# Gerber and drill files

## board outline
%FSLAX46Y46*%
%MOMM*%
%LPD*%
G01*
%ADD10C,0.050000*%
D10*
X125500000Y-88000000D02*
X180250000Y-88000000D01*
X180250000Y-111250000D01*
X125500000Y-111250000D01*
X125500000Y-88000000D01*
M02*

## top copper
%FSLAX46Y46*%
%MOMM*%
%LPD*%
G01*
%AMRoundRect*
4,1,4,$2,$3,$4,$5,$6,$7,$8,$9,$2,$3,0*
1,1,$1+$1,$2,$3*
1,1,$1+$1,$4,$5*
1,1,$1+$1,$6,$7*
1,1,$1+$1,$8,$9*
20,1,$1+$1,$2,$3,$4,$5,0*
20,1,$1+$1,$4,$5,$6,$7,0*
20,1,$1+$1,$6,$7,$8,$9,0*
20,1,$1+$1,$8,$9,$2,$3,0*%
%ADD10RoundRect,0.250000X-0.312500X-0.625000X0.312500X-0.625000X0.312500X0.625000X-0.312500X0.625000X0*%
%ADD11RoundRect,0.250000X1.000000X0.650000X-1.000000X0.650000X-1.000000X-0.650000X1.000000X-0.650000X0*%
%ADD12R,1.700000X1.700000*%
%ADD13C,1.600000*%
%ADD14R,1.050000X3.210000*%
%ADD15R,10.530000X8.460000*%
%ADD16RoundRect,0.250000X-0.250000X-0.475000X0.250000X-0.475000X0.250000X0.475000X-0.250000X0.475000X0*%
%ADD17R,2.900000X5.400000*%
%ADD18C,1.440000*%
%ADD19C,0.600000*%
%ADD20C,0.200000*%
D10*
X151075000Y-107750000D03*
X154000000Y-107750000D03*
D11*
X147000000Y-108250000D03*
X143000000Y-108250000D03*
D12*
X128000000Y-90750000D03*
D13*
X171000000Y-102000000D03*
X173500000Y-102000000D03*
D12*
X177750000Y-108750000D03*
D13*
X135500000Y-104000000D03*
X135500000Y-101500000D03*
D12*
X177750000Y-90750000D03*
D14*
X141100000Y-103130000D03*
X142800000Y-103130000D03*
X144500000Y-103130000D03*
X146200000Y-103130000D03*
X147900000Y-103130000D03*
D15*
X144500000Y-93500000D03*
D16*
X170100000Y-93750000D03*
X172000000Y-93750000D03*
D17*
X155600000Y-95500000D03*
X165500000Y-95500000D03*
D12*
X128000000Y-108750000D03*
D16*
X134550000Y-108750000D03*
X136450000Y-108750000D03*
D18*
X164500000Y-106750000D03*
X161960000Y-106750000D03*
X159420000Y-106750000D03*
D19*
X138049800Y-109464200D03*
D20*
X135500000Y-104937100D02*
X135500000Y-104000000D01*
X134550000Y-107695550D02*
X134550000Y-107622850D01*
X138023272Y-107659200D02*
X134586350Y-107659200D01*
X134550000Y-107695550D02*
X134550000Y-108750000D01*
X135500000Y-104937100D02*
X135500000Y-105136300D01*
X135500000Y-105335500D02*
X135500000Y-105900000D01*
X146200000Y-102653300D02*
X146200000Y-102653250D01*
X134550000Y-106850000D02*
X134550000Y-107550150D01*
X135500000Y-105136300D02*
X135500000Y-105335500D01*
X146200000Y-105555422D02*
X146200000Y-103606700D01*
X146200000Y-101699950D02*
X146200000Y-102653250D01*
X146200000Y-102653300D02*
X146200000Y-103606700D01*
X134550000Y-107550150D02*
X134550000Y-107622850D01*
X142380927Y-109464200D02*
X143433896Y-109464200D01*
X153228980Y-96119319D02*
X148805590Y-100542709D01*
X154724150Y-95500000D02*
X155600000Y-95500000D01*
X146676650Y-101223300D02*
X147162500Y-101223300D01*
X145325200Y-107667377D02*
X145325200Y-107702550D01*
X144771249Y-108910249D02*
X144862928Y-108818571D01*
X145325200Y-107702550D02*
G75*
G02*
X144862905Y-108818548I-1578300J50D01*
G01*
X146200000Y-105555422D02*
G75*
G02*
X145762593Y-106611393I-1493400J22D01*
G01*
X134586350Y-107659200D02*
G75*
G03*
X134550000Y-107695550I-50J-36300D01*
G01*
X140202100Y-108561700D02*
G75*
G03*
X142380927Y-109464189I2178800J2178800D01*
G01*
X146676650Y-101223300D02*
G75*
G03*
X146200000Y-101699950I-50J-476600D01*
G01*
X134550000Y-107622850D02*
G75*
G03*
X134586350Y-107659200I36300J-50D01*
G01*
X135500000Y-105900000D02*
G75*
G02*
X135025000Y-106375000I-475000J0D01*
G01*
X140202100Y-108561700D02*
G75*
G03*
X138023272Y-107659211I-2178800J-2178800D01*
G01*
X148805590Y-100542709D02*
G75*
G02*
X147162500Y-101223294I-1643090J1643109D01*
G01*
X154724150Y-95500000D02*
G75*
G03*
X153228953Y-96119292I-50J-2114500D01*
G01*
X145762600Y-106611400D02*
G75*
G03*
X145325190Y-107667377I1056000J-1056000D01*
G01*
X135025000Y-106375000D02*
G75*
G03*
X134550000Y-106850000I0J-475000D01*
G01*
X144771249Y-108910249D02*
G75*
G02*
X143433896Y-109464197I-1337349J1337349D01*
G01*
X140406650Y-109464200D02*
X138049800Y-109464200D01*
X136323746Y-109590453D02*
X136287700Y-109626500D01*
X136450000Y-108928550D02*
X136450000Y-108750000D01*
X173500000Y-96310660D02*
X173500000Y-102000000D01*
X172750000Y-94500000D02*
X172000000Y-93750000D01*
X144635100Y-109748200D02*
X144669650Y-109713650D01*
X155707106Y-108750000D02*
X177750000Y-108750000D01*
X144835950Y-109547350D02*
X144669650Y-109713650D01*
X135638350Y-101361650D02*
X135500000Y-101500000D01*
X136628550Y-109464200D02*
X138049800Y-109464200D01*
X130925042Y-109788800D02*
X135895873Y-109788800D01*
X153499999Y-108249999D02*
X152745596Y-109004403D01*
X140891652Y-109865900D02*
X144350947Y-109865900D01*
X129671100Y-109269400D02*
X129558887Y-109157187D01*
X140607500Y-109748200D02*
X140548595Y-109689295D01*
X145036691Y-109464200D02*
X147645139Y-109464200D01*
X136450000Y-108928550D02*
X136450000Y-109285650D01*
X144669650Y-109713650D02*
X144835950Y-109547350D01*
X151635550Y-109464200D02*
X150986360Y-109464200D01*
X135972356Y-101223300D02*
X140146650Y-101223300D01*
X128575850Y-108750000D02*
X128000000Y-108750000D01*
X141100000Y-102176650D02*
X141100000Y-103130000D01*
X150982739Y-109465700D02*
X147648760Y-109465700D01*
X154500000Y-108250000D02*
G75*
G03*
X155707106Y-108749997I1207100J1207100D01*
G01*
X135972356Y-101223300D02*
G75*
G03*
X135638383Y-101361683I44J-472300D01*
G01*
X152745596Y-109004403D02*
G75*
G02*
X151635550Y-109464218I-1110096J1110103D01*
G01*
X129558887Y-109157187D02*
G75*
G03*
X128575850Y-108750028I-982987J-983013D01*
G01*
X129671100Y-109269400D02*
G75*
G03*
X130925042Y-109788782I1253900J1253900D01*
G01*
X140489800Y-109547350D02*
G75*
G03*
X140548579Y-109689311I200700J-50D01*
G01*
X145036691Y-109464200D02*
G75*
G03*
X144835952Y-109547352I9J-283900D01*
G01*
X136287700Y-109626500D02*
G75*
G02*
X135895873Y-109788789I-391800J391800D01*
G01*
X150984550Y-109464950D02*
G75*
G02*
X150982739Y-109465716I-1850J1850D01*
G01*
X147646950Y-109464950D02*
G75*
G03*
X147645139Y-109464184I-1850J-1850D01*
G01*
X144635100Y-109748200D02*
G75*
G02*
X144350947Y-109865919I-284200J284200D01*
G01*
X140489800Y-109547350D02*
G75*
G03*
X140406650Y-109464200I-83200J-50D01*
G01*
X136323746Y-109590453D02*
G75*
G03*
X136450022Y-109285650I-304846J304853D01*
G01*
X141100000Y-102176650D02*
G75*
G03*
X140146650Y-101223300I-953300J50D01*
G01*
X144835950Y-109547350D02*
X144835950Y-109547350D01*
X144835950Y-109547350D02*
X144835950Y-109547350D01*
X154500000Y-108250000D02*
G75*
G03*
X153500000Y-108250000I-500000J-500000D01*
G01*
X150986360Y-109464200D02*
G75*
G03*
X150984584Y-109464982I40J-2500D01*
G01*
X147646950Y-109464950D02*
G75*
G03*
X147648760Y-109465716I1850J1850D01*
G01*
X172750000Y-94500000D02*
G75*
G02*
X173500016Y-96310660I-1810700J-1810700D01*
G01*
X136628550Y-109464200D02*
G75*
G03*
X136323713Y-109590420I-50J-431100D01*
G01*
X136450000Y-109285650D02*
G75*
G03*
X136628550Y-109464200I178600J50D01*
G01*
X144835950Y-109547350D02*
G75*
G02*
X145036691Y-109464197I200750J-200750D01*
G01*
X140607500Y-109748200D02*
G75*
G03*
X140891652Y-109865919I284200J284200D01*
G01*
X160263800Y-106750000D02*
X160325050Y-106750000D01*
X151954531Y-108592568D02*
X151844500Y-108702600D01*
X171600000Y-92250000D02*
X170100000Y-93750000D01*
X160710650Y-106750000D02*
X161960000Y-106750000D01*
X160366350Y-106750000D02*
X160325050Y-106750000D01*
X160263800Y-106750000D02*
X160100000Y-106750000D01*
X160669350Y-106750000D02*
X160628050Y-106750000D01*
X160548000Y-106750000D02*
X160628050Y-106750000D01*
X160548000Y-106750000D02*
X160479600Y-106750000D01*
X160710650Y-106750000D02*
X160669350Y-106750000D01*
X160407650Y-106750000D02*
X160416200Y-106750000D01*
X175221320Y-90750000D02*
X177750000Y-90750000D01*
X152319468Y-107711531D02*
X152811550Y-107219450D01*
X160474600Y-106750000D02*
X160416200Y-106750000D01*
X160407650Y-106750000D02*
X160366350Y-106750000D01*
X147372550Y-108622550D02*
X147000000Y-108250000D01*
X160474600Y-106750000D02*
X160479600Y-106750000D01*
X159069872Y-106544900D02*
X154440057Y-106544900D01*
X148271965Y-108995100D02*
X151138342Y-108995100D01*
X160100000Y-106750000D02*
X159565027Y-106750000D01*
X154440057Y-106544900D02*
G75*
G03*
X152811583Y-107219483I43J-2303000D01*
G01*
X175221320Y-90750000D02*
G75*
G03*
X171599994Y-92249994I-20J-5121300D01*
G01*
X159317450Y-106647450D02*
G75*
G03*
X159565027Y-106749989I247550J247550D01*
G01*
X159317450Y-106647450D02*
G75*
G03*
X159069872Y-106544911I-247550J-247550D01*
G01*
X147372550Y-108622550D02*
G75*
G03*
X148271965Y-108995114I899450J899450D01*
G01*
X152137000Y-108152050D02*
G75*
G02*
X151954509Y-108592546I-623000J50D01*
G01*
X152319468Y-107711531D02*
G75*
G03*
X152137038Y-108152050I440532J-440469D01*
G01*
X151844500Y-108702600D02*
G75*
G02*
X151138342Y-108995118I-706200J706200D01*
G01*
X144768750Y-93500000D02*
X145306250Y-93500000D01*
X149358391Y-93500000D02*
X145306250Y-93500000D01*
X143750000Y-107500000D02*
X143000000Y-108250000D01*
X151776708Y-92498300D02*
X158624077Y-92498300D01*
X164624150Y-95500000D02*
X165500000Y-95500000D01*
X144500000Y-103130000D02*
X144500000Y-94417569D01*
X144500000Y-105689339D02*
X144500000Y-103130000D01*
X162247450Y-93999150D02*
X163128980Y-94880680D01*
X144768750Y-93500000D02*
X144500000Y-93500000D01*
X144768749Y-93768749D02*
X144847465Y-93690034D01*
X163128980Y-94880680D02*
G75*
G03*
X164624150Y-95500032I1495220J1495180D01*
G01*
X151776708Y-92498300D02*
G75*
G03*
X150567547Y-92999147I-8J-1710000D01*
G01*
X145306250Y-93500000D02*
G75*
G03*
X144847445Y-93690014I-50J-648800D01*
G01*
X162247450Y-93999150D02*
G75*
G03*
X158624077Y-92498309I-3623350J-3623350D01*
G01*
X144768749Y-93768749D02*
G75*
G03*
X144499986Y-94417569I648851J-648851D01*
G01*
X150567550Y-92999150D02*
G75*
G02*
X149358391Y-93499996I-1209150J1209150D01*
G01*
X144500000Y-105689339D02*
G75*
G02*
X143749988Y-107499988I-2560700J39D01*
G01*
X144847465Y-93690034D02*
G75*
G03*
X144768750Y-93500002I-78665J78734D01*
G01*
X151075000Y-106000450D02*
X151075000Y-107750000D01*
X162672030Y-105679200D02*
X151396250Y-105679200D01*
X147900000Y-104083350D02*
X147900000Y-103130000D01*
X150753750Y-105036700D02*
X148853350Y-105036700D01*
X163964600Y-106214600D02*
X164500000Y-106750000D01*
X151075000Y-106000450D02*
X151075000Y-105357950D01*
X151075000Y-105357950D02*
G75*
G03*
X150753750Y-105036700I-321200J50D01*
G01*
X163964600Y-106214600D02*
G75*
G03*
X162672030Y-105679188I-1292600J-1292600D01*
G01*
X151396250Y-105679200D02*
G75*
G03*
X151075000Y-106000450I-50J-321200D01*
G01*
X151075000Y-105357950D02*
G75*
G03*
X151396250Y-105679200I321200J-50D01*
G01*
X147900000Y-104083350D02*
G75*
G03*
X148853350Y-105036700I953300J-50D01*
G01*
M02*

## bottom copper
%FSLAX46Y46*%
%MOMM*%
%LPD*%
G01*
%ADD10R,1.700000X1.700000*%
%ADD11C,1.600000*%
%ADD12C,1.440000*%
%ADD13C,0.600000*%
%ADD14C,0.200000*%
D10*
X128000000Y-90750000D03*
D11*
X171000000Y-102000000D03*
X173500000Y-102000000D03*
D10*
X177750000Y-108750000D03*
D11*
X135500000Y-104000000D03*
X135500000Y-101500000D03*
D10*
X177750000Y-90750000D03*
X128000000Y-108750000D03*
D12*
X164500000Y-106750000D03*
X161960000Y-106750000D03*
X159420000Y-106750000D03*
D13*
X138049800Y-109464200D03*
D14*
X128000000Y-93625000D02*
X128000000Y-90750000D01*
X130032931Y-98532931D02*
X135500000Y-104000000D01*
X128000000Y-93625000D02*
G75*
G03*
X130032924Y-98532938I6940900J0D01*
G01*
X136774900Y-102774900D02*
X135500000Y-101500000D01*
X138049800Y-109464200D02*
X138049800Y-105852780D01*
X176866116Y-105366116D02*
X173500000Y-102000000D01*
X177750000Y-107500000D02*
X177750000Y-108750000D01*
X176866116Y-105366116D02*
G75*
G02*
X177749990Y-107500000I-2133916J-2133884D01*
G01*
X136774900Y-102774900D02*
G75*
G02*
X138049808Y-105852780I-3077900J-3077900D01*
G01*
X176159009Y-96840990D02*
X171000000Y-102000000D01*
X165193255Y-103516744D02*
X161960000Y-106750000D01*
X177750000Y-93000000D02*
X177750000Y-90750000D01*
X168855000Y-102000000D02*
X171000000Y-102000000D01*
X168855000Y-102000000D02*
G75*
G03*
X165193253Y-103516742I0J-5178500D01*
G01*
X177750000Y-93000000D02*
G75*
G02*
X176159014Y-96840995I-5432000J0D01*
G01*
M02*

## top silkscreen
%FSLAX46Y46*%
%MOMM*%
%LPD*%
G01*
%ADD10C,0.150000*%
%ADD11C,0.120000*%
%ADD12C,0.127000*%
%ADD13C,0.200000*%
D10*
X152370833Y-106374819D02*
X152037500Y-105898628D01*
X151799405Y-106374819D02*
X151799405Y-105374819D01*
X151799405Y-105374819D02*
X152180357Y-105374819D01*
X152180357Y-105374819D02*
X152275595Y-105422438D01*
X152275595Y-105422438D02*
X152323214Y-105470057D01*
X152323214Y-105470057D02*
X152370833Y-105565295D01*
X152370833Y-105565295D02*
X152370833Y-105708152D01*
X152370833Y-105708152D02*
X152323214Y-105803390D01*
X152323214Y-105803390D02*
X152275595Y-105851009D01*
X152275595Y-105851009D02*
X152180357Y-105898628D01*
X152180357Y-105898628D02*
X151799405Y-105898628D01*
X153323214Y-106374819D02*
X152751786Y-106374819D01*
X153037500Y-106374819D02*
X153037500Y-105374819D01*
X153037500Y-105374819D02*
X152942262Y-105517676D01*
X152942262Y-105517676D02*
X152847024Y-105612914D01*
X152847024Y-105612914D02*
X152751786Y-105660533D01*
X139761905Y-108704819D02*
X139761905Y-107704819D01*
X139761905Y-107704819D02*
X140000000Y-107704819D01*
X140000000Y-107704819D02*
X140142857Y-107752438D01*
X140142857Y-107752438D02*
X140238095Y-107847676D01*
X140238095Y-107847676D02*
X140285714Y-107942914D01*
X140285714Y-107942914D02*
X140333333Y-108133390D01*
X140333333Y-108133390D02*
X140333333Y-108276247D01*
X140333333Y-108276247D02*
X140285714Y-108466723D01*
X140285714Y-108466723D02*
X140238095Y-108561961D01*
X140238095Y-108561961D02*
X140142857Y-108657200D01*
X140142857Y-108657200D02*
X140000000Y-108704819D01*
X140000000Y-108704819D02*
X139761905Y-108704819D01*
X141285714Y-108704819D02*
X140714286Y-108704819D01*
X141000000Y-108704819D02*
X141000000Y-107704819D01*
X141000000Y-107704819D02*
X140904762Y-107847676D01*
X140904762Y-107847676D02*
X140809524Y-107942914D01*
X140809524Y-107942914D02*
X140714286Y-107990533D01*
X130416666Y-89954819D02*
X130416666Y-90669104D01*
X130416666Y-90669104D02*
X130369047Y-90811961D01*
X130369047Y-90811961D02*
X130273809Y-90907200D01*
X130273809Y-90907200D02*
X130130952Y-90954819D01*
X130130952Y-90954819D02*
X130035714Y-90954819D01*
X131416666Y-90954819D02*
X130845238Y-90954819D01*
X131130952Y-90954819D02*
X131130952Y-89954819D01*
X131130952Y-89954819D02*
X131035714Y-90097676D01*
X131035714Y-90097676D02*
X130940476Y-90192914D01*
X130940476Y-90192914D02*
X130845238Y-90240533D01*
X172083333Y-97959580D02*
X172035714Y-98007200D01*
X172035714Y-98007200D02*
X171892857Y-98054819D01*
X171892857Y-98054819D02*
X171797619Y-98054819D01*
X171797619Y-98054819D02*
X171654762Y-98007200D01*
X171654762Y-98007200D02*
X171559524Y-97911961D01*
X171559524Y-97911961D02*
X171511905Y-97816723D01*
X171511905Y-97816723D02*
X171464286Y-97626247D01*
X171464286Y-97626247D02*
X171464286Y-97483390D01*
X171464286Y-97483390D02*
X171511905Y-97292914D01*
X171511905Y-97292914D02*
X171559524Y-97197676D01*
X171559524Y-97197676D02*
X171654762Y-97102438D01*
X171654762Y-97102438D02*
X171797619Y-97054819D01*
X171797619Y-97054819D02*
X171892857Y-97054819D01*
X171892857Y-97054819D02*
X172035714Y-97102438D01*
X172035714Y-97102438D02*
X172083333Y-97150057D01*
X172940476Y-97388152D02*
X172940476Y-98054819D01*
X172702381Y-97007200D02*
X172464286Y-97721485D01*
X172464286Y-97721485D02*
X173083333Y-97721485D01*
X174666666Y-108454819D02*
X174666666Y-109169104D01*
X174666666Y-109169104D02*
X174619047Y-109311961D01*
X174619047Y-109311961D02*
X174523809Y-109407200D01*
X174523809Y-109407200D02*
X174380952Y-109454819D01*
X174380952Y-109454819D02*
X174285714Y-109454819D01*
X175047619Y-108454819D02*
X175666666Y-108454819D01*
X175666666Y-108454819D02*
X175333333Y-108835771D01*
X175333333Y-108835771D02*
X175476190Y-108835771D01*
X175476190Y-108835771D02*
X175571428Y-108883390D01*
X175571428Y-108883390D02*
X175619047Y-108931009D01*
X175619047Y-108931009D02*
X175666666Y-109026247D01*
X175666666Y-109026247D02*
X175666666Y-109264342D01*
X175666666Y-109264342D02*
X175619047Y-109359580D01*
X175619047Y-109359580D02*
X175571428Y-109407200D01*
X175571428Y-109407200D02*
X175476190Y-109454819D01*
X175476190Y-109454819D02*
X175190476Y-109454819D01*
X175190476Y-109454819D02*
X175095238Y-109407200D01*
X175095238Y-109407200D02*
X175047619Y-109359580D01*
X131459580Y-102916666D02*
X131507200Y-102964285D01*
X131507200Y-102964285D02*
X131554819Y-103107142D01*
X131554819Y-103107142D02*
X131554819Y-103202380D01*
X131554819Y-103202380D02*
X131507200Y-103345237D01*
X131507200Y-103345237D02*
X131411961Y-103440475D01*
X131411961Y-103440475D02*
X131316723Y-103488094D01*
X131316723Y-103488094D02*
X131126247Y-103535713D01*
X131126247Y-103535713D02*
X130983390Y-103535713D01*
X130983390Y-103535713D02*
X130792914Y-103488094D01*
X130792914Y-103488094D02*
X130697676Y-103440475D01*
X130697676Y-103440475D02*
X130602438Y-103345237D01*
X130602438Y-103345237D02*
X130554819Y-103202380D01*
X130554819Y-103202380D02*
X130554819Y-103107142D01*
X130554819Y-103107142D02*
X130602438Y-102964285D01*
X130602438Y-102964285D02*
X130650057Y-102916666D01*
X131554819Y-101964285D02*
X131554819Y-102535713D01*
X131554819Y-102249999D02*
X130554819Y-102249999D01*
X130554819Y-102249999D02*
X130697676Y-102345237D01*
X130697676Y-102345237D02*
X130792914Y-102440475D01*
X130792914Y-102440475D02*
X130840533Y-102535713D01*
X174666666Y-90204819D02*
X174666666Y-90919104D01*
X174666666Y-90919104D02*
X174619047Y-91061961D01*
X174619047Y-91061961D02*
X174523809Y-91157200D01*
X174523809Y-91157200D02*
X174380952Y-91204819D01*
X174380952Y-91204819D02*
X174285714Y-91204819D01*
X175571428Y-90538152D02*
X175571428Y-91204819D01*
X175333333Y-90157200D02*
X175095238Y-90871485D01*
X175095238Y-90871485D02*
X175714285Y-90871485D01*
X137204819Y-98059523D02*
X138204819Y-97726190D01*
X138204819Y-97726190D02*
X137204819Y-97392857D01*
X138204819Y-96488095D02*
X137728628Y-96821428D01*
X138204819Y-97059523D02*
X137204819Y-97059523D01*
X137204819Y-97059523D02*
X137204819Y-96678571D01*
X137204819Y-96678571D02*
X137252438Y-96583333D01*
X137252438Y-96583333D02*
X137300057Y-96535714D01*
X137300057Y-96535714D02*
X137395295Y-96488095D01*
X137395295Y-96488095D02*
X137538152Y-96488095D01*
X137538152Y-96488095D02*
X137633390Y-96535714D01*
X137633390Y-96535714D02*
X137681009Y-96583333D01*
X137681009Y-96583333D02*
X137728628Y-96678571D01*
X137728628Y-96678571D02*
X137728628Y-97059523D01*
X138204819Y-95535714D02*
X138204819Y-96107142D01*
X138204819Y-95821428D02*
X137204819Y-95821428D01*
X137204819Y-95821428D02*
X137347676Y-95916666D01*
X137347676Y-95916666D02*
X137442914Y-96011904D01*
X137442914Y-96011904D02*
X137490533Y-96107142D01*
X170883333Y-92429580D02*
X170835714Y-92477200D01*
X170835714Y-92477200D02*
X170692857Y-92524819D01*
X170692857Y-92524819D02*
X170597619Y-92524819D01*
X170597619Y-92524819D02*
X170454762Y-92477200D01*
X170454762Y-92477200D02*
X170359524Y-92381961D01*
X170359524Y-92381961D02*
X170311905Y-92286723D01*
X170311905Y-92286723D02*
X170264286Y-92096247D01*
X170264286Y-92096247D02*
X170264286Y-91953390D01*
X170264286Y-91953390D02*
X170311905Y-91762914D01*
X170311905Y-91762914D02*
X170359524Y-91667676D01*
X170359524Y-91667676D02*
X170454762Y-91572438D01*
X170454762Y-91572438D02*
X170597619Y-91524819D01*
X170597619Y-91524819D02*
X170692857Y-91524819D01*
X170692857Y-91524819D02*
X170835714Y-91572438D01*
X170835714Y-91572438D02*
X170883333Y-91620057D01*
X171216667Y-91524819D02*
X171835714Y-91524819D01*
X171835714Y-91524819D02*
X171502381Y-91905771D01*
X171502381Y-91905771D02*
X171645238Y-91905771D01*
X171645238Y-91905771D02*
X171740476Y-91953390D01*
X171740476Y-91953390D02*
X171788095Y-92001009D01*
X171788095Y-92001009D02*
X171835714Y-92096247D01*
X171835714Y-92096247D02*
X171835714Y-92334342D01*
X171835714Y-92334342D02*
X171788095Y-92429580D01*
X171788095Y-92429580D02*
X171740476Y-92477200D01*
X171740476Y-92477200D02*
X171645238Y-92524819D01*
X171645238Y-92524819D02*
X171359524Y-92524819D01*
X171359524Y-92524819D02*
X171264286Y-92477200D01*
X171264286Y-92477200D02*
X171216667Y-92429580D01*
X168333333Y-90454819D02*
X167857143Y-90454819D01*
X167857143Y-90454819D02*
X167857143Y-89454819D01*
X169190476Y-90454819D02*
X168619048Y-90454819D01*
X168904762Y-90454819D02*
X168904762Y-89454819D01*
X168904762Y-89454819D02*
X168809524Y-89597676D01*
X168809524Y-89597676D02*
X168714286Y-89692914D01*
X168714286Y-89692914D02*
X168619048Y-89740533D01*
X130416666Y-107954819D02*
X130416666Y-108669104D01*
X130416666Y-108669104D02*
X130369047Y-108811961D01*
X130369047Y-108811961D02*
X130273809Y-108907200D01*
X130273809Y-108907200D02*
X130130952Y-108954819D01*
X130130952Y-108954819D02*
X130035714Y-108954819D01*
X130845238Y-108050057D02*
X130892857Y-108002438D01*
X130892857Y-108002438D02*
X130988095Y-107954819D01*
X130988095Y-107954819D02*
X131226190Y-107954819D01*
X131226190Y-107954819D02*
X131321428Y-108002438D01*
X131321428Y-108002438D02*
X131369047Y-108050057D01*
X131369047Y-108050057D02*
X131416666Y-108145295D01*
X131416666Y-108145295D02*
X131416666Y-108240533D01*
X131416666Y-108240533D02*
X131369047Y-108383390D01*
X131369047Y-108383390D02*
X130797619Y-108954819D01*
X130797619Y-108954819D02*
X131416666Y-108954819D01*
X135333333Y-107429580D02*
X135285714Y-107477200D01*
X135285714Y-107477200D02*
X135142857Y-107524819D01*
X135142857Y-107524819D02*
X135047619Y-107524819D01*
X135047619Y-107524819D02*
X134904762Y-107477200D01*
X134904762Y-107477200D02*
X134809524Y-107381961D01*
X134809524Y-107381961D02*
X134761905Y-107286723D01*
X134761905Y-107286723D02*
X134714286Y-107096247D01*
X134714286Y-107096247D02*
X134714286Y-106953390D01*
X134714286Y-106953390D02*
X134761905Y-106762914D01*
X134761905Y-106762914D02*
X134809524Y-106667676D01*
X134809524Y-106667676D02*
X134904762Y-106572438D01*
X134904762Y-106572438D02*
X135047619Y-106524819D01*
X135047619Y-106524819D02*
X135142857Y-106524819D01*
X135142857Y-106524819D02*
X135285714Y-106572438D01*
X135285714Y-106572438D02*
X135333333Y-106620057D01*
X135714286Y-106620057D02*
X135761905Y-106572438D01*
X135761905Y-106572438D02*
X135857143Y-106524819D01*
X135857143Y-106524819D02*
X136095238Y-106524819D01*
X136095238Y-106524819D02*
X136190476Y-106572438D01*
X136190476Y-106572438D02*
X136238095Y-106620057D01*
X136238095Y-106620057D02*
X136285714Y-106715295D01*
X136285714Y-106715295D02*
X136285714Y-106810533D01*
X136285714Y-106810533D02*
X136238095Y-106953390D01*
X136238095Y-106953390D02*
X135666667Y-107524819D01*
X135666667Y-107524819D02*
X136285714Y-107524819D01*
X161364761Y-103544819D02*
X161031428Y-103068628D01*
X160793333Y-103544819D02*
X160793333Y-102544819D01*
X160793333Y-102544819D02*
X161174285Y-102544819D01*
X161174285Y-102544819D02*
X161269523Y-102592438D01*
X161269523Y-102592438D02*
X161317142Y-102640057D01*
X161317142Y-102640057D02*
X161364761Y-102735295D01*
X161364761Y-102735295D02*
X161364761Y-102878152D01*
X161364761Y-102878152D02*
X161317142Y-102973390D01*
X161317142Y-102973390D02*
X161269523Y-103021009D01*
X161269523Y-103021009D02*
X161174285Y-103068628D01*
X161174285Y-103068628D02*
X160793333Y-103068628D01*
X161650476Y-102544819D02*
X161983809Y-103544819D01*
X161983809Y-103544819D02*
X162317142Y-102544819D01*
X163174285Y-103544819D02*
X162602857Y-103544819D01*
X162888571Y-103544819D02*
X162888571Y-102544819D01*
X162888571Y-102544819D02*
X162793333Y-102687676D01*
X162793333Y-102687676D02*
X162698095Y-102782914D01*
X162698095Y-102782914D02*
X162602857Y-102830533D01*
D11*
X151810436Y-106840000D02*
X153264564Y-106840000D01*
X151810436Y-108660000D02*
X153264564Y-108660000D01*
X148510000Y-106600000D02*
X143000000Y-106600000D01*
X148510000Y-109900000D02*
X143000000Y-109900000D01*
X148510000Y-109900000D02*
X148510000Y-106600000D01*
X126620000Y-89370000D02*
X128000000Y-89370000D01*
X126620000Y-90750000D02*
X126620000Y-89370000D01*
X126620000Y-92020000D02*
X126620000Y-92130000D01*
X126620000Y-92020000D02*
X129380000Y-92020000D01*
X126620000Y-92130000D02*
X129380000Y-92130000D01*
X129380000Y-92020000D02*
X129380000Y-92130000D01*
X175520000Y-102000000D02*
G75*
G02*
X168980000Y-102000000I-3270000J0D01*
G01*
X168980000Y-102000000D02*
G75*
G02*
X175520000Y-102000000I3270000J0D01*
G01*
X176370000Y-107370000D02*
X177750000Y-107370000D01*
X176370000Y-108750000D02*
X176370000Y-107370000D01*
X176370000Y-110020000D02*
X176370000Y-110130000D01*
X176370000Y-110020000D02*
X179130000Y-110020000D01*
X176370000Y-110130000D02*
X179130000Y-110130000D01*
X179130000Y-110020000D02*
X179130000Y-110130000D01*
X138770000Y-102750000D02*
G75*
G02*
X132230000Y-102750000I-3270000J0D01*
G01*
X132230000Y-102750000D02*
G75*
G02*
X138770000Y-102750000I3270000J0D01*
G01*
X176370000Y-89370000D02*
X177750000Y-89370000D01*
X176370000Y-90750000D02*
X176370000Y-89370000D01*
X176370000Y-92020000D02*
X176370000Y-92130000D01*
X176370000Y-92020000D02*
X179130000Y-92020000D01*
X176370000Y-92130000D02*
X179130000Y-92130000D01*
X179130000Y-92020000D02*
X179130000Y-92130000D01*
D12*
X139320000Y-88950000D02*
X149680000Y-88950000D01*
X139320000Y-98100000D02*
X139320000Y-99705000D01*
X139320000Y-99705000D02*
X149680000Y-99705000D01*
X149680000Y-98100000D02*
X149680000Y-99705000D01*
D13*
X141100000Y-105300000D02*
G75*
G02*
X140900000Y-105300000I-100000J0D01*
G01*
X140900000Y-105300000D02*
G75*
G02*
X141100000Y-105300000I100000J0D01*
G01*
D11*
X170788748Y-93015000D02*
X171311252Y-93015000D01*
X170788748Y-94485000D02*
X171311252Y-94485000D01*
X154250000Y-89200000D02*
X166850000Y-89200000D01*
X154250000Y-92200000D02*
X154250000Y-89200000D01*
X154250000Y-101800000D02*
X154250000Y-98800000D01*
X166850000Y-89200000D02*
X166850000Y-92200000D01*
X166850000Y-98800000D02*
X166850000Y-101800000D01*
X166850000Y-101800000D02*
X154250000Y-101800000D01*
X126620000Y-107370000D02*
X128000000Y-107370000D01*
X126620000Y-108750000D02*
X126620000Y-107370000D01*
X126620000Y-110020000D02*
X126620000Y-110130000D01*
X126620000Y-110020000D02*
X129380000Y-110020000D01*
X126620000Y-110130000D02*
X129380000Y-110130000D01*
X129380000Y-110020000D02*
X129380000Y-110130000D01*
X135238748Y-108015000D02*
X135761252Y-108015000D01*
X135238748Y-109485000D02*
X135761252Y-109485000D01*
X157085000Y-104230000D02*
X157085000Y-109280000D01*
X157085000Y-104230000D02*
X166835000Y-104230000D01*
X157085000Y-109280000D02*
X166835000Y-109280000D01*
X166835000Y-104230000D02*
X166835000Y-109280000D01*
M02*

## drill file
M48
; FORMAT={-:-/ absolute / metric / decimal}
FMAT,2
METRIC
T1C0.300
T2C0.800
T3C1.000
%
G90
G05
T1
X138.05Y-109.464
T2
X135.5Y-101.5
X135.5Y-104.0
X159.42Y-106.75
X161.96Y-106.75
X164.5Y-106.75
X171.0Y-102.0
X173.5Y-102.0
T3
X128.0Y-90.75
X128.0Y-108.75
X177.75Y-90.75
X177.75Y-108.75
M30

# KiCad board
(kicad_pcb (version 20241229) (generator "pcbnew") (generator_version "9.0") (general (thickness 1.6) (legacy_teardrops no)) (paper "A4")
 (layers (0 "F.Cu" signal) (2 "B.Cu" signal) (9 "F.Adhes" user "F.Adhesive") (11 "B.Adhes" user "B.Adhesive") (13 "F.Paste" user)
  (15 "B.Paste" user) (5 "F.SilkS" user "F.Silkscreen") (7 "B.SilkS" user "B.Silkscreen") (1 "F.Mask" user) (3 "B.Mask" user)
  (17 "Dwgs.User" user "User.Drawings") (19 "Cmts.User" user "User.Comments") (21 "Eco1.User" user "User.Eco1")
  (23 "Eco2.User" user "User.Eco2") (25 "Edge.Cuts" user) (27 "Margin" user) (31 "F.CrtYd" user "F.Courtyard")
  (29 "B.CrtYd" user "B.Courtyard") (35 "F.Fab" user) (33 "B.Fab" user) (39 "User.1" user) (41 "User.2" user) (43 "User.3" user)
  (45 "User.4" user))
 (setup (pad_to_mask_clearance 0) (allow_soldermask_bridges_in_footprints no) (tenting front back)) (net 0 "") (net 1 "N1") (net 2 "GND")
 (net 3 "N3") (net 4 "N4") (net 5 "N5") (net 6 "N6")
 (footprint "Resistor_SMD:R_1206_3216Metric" (layer "F.Cu") (at 152.5375 107.75)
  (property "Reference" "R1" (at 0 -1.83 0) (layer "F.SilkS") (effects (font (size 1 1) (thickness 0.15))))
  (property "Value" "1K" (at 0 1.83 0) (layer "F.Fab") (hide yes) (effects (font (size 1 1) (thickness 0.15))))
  (fp_line (start -0.727064 -0.91) (end 0.727064 -0.91) (stroke (width 0.12) (type solid)) (layer "F.SilkS"))
  (fp_line (start -0.727064 0.91) (end 0.727064 0.91) (stroke (width 0.12) (type solid)) (layer "F.SilkS"))
  (pad "1" smd roundrect (at -1.4625 0) (size 1.125 1.75) (layers "F.Cu" "F.Mask" "F.Paste") (roundrect_rratio 0.222222) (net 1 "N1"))
  (pad "2" smd roundrect (at 1.4625 0) (size 1.125 1.75) (layers "F.Cu" "F.Mask" "F.Paste") (roundrect_rratio 0.222222) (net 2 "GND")))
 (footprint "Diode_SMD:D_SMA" (layer "F.Cu") (at 145 108.25 180)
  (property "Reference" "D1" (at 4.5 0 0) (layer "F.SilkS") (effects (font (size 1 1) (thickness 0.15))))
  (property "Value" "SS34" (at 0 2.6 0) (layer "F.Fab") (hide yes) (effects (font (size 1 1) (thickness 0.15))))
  (fp_line (start -3.51 1.65) (end 2 1.65) (stroke (width 0.12) (type solid)) (layer "F.SilkS"))
  (fp_line (start -3.51 -1.65) (end 2 -1.65) (stroke (width 0.12) (type solid)) (layer "F.SilkS"))
  (fp_line (start -3.51 -1.65) (end -3.51 1.65) (stroke (width 0.12) (type solid)) (layer "F.SilkS"))
  (pad "1" smd roundrect (at -2 0 180) (size 2.5 1.8) (layers "F.Cu" "F.Mask" "F.Paste") (roundrect_rratio 0.1388888889) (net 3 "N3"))
  (pad "2" smd roundrect (at 2 0 180) (size 2.5 1.8) (layers "F.Cu" "F.Mask" "F.Paste") (roundrect_rratio 0.1388888889) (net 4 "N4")))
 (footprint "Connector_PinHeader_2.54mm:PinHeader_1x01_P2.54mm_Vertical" (layer "F.Cu") (at 128 90.75)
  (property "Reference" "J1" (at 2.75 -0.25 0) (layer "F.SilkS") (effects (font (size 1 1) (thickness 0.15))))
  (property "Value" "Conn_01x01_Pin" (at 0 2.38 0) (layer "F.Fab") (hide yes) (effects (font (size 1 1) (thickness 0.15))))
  (fp_line (start -1.38 -1.38) (end 0 -1.38) (stroke (width 0.12) (type solid)) (layer "F.SilkS"))
  (fp_line (start -1.38 0) (end -1.38 -1.38) (stroke (width 0.12) (type solid)) (layer "F.SilkS"))
  (fp_line (start -1.38 1.27) (end -1.38 1.38) (stroke (width 0.12) (type solid)) (layer "F.SilkS"))
  (fp_line (start -1.38 1.27) (end 1.38 1.27) (stroke (width 0.12) (type solid)) (layer "F.SilkS"))
  (fp_line (start -1.38 1.38) (end 1.38 1.38) (stroke (width 0.12) (type solid)) (layer "F.SilkS"))
  (fp_line (start 1.38 1.27) (end 1.38 1.38) (stroke (width 0.12) (type solid)) (layer "F.SilkS"))
  (pad "1" thru_hole rect (at 0 0) (size 1.7 1.7) (drill 1) (layers "*.Cu" "*.Mask") (remove_unused_layers no) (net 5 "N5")))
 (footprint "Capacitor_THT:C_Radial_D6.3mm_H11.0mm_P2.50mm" (layer "F.Cu") (at 171 102)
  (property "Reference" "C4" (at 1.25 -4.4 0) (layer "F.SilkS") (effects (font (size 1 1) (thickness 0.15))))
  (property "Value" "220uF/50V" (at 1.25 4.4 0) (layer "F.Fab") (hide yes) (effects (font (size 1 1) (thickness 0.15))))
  (fp_circle (center 1.25 0) (end 4.52 0) (stroke (width 0.12) (type solid)) (fill no) (layer "F.SilkS"))
  (pad "1" thru_hole circle (at 0 0) (size 1.6 1.6) (drill 0.8) (layers "*.Cu" "*.Mask") (remove_unused_layers no) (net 3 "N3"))
  (pad "2" thru_hole circle (at 2.5 0) (size 1.6 1.6) (drill 0.8) (layers "*.Cu" "*.Mask") (remove_unused_layers no) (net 2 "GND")))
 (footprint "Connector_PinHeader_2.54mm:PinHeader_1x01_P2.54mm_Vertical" (layer "F.Cu") (at 177.75 108.75)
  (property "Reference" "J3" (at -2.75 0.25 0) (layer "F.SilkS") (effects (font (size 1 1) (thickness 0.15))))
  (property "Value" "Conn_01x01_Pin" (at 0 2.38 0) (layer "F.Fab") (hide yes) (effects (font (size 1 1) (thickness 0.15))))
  (fp_line (start -1.38 -1.38) (end 0 -1.38) (stroke (width 0.12) (type solid)) (layer "F.SilkS"))
  (fp_line (start -1.38 0) (end -1.38 -1.38) (stroke (width 0.12) (type solid)) (layer "F.SilkS"))
  (fp_line (start -1.38 1.27) (end -1.38 1.38) (stroke (width 0.12) (type solid)) (layer "F.SilkS"))
  (fp_line (start -1.38 1.27) (end 1.38 1.27) (stroke (width 0.12) (type solid)) (layer "F.SilkS"))
  (fp_line (start -1.38 1.38) (end 1.38 1.38) (stroke (width 0.12) (type solid)) (layer "F.SilkS"))
  (fp_line (start 1.38 1.27) (end 1.38 1.38) (stroke (width 0.12) (type solid)) (layer "F.SilkS"))
  (pad "1" thru_hole rect (at 0 0) (size 1.7 1.7) (drill 1) (layers "*.Cu" "*.Mask") (remove_unused_layers no) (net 2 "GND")))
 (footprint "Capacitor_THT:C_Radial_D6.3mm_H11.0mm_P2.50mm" (layer "F.Cu") (at 135.5 104 90)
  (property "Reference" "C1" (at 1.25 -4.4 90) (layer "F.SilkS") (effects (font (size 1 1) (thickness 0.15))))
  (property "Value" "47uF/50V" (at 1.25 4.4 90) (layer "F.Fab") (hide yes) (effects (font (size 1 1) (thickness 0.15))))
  (fp_circle (center 1.25 0) (end 4.52 0) (stroke (width 0.12) (type solid)) (fill no) (layer "F.SilkS"))
  (pad "1" thru_hole circle (at 0 0 90) (size 1.6 1.6) (drill 0.8) (layers "*.Cu" "*.Mask") (remove_unused_layers no) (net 5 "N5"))
  (pad "2" thru_hole circle (at 2.5 0 90) (size 1.6 1.6) (drill 0.8) (layers "*.Cu" "*.Mask") (remove_unused_layers no) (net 2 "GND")))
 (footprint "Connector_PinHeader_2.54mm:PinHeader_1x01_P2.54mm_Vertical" (layer "F.Cu") (at 177.75 90.75)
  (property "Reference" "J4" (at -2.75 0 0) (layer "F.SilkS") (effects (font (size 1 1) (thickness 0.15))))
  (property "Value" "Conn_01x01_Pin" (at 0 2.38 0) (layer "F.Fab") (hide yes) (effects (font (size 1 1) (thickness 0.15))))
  (fp_line (start -1.38 -1.38) (end 0 -1.38) (stroke (width 0.12) (type solid)) (layer "F.SilkS"))
  (fp_line (start -1.38 0) (end -1.38 -1.38) (stroke (width 0.12) (type solid)) (layer "F.SilkS"))
  (fp_line (start -1.38 1.27) (end -1.38 1.38) (stroke (width 0.12) (type solid)) (layer "F.SilkS"))
  (fp_line (start -1.38 1.27) (end 1.38 1.27) (stroke (width 0.12) (type solid)) (layer "F.SilkS"))
  (fp_line (start -1.38 1.38) (end 1.38 1.38) (stroke (width 0.12) (type solid)) (layer "F.SilkS"))
  (fp_line (start 1.38 1.27) (end 1.38 1.38) (stroke (width 0.12) (type solid)) (layer "F.SilkS"))
  (pad "1" thru_hole rect (at 0 0) (size 1.7 1.7) (drill 1) (layers "*.Cu" "*.Mask") (remove_unused_layers no) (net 3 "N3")))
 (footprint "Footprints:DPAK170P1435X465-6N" (layer "F.Cu") (at 144.5 97 90)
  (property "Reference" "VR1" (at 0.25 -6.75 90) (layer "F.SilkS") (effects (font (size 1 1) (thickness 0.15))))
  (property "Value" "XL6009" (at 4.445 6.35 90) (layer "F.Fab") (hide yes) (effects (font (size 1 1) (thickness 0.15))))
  (fp_line (start 8.05 -5.18) (end 8.05 5.18) (stroke (width 0.127) (type solid)) (layer "F.SilkS"))
  (fp_line (start -1.1 -5.18) (end -2.705 -5.18) (stroke (width 0.127) (type solid)) (layer "F.SilkS"))
  (fp_line (start -2.705 -5.18) (end -2.705 5.18) (stroke (width 0.127) (type solid)) (layer "F.SilkS"))
  (fp_line (start -1.1 5.18) (end -2.705 5.18) (stroke (width 0.127) (type solid)) (layer "F.SilkS"))
  (fp_circle (center -8.3 -3.5) (end -8.2 -3.5) (stroke (width 0.2) (type solid)) (fill no) (layer "F.SilkS"))
  (pad "1" smd rect (at -6.13 -3.4 90) (size 3.21 1.05) (layers "F.Cu" "F.Mask" "F.Paste") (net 2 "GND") (solder_mask_margin 0.102))
  (pad "2" smd rect (at -6.13 -1.7 90) (size 3.21 1.05) (layers "F.Cu" "F.Mask" "F.Paste") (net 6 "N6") (solder_mask_margin 0.102))
  (pad "3" smd rect (at -6.13 0 90) (size 3.21 1.05) (layers "F.Cu" "F.Mask" "F.Paste") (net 4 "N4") (solder_mask_margin 0.102))
  (pad "4" smd rect (at -6.13 1.7 90) (size 3.21 1.05) (layers "F.Cu" "F.Mask" "F.Paste") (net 5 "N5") (solder_mask_margin 0.102))
  (pad "5" smd rect (at -6.13 3.4 90) (size 3.21 1.05) (layers "F.Cu" "F.Mask" "F.Paste") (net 1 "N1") (solder_mask_margin 0.102))
  (pad "6" smd rect (at 3.5 0 90) (size 8.46 10.53) (layers "F.Cu" "F.Mask") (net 4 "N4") (solder_mask_margin 0.102)))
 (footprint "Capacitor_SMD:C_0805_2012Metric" (layer "F.Cu") (at 171.05 93.75)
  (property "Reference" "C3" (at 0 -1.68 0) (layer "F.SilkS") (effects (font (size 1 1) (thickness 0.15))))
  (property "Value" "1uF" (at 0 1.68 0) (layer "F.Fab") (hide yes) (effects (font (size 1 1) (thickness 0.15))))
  (fp_line (start -0.261252 -0.735) (end 0.261252 -0.735) (stroke (width 0.12) (type solid)) (layer "F.SilkS"))
  (fp_line (start -0.261252 0.735) (end 0.261252 0.735) (stroke (width 0.12) (type solid)) (layer "F.SilkS"))
  (pad "1" smd roundrect (at -0.95 0) (size 1 1.45) (layers "F.Cu" "F.Mask" "F.Paste") (roundrect_rratio 0.25) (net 3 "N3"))
  (pad "2" smd roundrect (at 0.95 0) (size 1 1.45) (layers "F.Cu" "F.Mask" "F.Paste") (roundrect_rratio 0.25) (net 2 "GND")))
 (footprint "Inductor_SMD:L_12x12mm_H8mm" (layer "F.Cu") (at 160.55 95.5)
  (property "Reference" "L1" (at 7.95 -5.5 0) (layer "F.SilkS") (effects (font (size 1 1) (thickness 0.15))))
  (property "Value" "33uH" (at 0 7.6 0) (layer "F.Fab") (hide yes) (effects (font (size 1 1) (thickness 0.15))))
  (fp_line (start -6.3 -6.3) (end 6.3 -6.3) (stroke (width 0.12) (type solid)) (layer "F.SilkS"))
  (fp_line (start -6.3 -3.3) (end -6.3 -6.3) (stroke (width 0.12) (type solid)) (layer "F.SilkS"))
  (fp_line (start -6.3 6.3) (end -6.3 3.3) (stroke (width 0.12) (type solid)) (layer "F.SilkS"))
  (fp_line (start 6.3 -6.3) (end 6.3 -3.3) (stroke (width 0.12) (type solid)) (layer "F.SilkS"))
  (fp_line (start 6.3 3.3) (end 6.3 6.3) (stroke (width 0.12) (type solid)) (layer "F.SilkS"))
  (fp_line (start 6.3 6.3) (end -6.3 6.3) (stroke (width 0.12) (type solid)) (layer "F.SilkS"))
  (pad "1" smd rect (at -4.95 0) (size 2.9 5.4) (layers "F.Cu" "F.Mask" "F.Paste") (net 5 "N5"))
  (pad "2" smd rect (at 4.95 0) (size 2.9 5.4) (layers "F.Cu" "F.Mask" "F.Paste") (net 4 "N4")))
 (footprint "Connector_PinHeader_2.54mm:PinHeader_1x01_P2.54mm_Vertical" (layer "F.Cu") (at 128 108.75)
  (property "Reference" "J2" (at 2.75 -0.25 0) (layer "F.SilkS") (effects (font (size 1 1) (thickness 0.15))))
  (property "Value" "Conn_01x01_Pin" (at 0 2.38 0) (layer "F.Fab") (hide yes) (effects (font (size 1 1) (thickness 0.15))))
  (fp_line (start -1.38 -1.38) (end 0 -1.38) (stroke (width 0.12) (type solid)) (layer "F.SilkS"))
  (fp_line (start -1.38 0) (end -1.38 -1.38) (stroke (width 0.12) (type solid)) (layer "F.SilkS"))
  (fp_line (start -1.38 1.27) (end -1.38 1.38) (stroke (width 0.12) (type solid)) (layer "F.SilkS"))
  (fp_line (start -1.38 1.27) (end 1.38 1.27) (stroke (width 0.12) (type solid)) (layer "F.SilkS"))
  (fp_line (start -1.38 1.38) (end 1.38 1.38) (stroke (width 0.12) (type solid)) (layer "F.SilkS"))
  (fp_line (start 1.38 1.27) (end 1.38 1.38) (stroke (width 0.12) (type solid)) (layer "F.SilkS"))
  (pad "1" thru_hole rect (at 0 0) (size 1.7 1.7) (drill 1) (layers "*.Cu" "*.Mask") (remove_unused_layers no) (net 2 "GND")))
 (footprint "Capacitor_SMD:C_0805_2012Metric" (layer "F.Cu") (at 135.5 108.75)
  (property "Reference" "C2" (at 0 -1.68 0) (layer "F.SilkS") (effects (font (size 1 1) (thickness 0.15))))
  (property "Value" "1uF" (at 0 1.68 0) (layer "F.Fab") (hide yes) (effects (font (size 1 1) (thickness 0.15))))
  (fp_line (start -0.261252 -0.735) (end 0.261252 -0.735) (stroke (width 0.12) (type solid)) (layer "F.SilkS"))
  (fp_line (start -0.261252 0.735) (end 0.261252 0.735) (stroke (width 0.12) (type solid)) (layer "F.SilkS"))
  (pad "1" smd roundrect (at -0.95 0) (size 1 1.45) (layers "F.Cu" "F.Mask" "F.Paste") (roundrect_rratio 0.25) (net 5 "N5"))
  (pad "2" smd roundrect (at 0.95 0) (size 1 1.45) (layers "F.Cu" "F.Mask" "F.Paste") (roundrect_rratio 0.25) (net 2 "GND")))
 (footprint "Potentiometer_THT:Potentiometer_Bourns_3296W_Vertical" (layer "F.Cu") (at 164.5 106.75)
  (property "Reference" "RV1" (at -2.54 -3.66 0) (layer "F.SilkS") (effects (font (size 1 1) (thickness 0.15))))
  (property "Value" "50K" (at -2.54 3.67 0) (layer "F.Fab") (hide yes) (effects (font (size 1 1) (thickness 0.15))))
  (fp_line (start -7.415 -2.52) (end -7.415 2.53) (stroke (width 0.12) (type solid)) (layer "F.SilkS"))
  (fp_line (start -7.415 -2.52) (end 2.335 -2.52) (stroke (width 0.12) (type solid)) (layer "F.SilkS"))
  (fp_line (start -7.415 2.53) (end 2.335 2.53) (stroke (width 0.12) (type solid)) (layer "F.SilkS"))
  (fp_line (start 2.335 -2.52) (end 2.335 2.53) (stroke (width 0.12) (type solid)) (layer "F.SilkS"))
  (pad "1" thru_hole circle (at 0 0) (size 1.44 1.44) (drill 0.8) (layers "*.Cu" "*.Mask") (remove_unused_layers no) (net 1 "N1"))
  (pad "2" thru_hole circle (at -2.54 0) (size 1.44 1.44) (drill 0.8) (layers "*.Cu" "*.Mask") (remove_unused_layers no) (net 3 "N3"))
  (pad "3" thru_hole circle (at -5.08 0) (size 1.44 1.44) (drill 0.8) (layers "*.Cu" "*.Mask") (remove_unused_layers no) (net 3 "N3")))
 (gr_rect (start 125.5 88) (end 180.25 111.25) (stroke (width 0.05) (type default)) (fill no) (layer "Edge.Cuts"))
 (segment (start 135.5 104.9371) (end 135.5 104) (width 0.2) (layer "F.Cu") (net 5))
 (segment (start 134.55 107.69555) (end 134.55 107.62285) (width 0.2) (layer "F.Cu") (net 5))
 (segment (start 138.023272 107.6592) (end 134.58635 107.6592) (width 0.2) (layer "F.Cu") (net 5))
 (segment (start 134.55 107.69555) (end 134.55 108.75) (width 0.2) (layer "F.Cu") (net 5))
 (segment (start 135.5 104.9371) (end 135.5 105.1363) (width 0.2) (layer "F.Cu") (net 5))
 (segment (start 135.5 105.3355) (end 135.5 105.9) (width 0.2) (layer "F.Cu") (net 5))
 (segment (start 146.2 102.6533) (end 146.2 102.65325) (width 0.2) (layer "F.Cu") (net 5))
 (segment (start 134.55 106.85) (end 134.55 107.55015) (width 0.2) (layer "F.Cu") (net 5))
 (segment (start 135.5 105.1363) (end 135.5 105.3355) (width 0.2) (layer "F.Cu") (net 5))
 (segment (start 146.2 105.555422) (end 146.2 103.6067) (width 0.2) (layer "F.Cu") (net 5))
 (segment (start 146.2 101.69995) (end 146.2 102.65325) (width 0.2) (layer "F.Cu") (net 5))
 (segment (start 146.2 102.6533) (end 146.2 103.6067) (width 0.2) (layer "F.Cu") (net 5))
 (segment (start 134.55 107.55015) (end 134.55 107.62285) (width 0.2) (layer "F.Cu") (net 5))
 (segment (start 142.380927 109.4642) (end 143.433896 109.4642) (width 0.2) (layer "F.Cu") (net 5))
 (segment (start 153.22898 96.119319) (end 148.80559 100.542709) (width 0.2) (layer "F.Cu") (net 5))
 (segment (start 154.72415 95.5) (end 155.6 95.5) (width 0.2) (layer "F.Cu") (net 5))
 (segment (start 146.67665 101.2233) (end 147.1625 101.2233) (width 0.2) (layer "F.Cu") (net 5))
 (segment (start 145.3252 107.667377) (end 145.3252 107.70255) (width 0.2) (layer "F.Cu") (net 5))
 (segment (start 144.771249 108.910249) (end 144.862928 108.818571) (width 0.2) (layer "F.Cu") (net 5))
 (arc (start 145.3252 107.70255) (mid 145.205059 108.306536) (end 144.862928 108.818571) (width 0.2) (layer "F.Cu") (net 5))
 (arc (start 146.2 105.555422) (mid 146.086323 106.126913) (end 145.7626 106.6114) (width 0.2) (layer "F.Cu") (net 5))
 (arc (start 134.58635 107.6592) (mid 134.560646 107.669846) (end 134.55 107.69555) (width 0.2) (layer "F.Cu") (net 5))
 (arc (start 140.2021 108.5617) (mid 141.201754 109.229647) (end 142.380927 109.4642) (width 0.2) (layer "F.Cu") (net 5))
 (arc (start 146.67665 101.2233) (mid 146.339607 101.362907) (end 146.2 101.69995) (width 0.2) (layer "F.Cu") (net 5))
 (arc (start 134.55 107.62285) (mid 134.560646 107.648553) (end 134.58635 107.6592) (width 0.2) (layer "F.Cu") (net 5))
 (arc (start 135.5 105.9) (mid 135.360875 106.235875) (end 135.025 106.375) (width 0.2) (layer "F.Cu") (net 5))
 (arc (start 140.2021 108.5617) (mid 139.202445 107.893752) (end 138.023272 107.6592) (width 0.2) (layer "F.Cu") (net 5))
 (arc (start 148.80559 100.542709) (mid 148.051733 101.04642) (end 147.1625 101.2233) (width 0.2) (layer "F.Cu") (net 5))
 (arc (start 154.72415 95.5) (mid 153.914969 95.660955) (end 153.22898 96.119319) (width 0.2) (layer "F.Cu") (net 5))
 (arc (start 145.7626 106.6114) (mid 145.438876 107.095886) (end 145.3252 107.667377) (width 0.2) (layer "F.Cu") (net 5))
 (arc (start 135.025 106.375) (mid 134.689124 106.514124) (end 134.55 106.85) (width 0.2) (layer "F.Cu") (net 5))
 (arc (start 144.771249 108.910249) (mid 144.157666 109.320232) (end 143.433896 109.4642) (width 0.2) (layer "F.Cu") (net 5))
 (segment (start 128 93.625) (end 128 90.75) (width 0.2) (layer "B.Cu") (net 5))
 (segment (start 130.032931 98.532931) (end 135.5 104) (width 0.2) (layer "B.Cu") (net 5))
 (arc (start 128 93.625) (mid 128.528341 96.281153) (end 130.032931 98.532931) (width 0.2) (layer "B.Cu") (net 5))
 (segment (start 140.40665 109.4642) (end 138.0498 109.4642) (width 0.2) (layer "F.Cu") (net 2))
 (segment (start 136.323746 109.590453) (end 136.2877 109.6265) (width 0.2) (layer "F.Cu") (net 2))
 (segment (start 136.45 108.92855) (end 136.45 108.75) (width 0.2) (layer "F.Cu") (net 2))
 (segment (start 173.5 96.31066) (end 173.5 102) (width 0.2) (layer "F.Cu") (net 2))
 (segment (start 172.75 94.5) (end 172 93.75) (width 0.2) (layer "F.Cu") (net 2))
 (segment (start 144.6351 109.7482) (end 144.66965 109.71365) (width 0.2) (layer "F.Cu") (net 2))
 (segment (start 155.707106 108.75) (end 177.75 108.75) (width 0.2) (layer "F.Cu") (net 2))
 (segment (start 144.83595 109.54735) (end 144.66965 109.71365) (width 0.2) (layer "F.Cu") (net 2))
 (segment (start 135.63835 101.36165) (end 135.5 101.5) (width 0.2) (layer "F.Cu") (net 2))
 (segment (start 136.62855 109.4642) (end 138.0498 109.4642) (width 0.2) (layer "F.Cu") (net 2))
 (segment (start 130.925042 109.7888) (end 135.895873 109.7888) (width 0.2) (layer "F.Cu") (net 2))
 (segment (start 153.499999 108.249999) (end 152.745596 109.004403) (width 0.2) (layer "F.Cu") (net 2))
 (segment (start 140.891652 109.8659) (end 144.350947 109.8659) (width 0.2) (layer "F.Cu") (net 2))
 (segment (start 129.6711 109.2694) (end 129.558887 109.157187) (width 0.2) (layer "F.Cu") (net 2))
 (segment (start 140.6075 109.7482) (end 140.548595 109.689295) (width 0.2) (layer "F.Cu") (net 2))
 (segment (start 145.036691 109.4642) (end 147.645139 109.4642) (width 0.2) (layer "F.Cu") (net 2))
 (segment (start 136.45 108.92855) (end 136.45 109.28565) (width 0.2) (layer "F.Cu") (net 2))
 (segment (start 144.66965 109.71365) (end 144.83595 109.54735) (width 0.2) (layer "F.Cu") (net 2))
 (segment (start 151.63555 109.4642) (end 150.98636 109.4642) (width 0.2) (layer "F.Cu") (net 2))
 (segment (start 135.972356 101.2233) (end 140.14665 101.2233) (width 0.2) (layer "F.Cu") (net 2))
 (segment (start 128.57585 108.75) (end 128 108.75) (width 0.2) (layer "F.Cu") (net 2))
 (segment (start 141.1 102.17665) (end 141.1 103.13) (width 0.2) (layer "F.Cu") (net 2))
 (segment (start 150.982739 109.4657) (end 147.64876 109.4657) (width 0.2) (layer "F.Cu") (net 2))
 (via (at 138.0498 109.4642) (size 0.6) (drill 0.3) (layers "F.Cu" "B.Cu") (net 2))
 (arc (start 154.5 108.25) (mid 155.053825 108.620054) (end 155.707106 108.75) (width 0.2) (layer "F.Cu") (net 2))
 (arc (start 135.972356 101.2233) (mid 135.791593 101.259255) (end 135.63835 101.36165) (width 0.2) (layer "F.Cu") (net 2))
 (arc (start 152.745596 109.004403) (mid 152.236302 109.344702) (end 151.63555 109.4642) (width 0.2) (layer "F.Cu") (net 2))
 (arc (start 129.558887 109.157187) (mid 129.107865 108.855824) (end 128.57585 108.75) (width 0.2) (layer "F.Cu") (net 2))
 (arc (start 129.6711 109.2694) (mid 130.246413 109.653812) (end 130.925042 109.7888) (width 0.2) (layer "F.Cu") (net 2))
 (arc (start 140.4898 109.54735) (mid 140.50508 109.62417) (end 140.548595 109.689295) (width 0.2) (layer "F.Cu") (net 2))
 (arc (start 145.036691 109.4642) (mid 144.92805 109.485809) (end 144.83595 109.54735) (width 0.2) (layer "F.Cu") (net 2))
 (arc (start 136.2877 109.6265) (mid 136.107928 109.746619) (end 135.895873 109.7888) (width 0.2) (layer "F.Cu") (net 2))
 (arc (start 150.98455 109.46495) (mid 150.983719 109.465505) (end 150.982739 109.4657) (width 0.2) (layer "F.Cu") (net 2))
 (arc (start 147.64695 109.46495) (mid 147.646119 109.464394) (end 147.645139 109.4642) (width 0.2) (layer "F.Cu") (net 2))
 (arc (start 144.6351 109.7482) (mid 144.504729 109.83531) (end 144.350947 109.8659) (width 0.2) (layer "F.Cu") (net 2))
 (arc (start 140.4898 109.54735) (mid 140.465445 109.488554) (end 140.40665 109.4642) (width 0.2) (layer "F.Cu") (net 2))
 (arc (start 136.323746 109.590453) (mid 136.417187 109.450608) (end 136.45 109.28565) (width 0.2) (layer "F.Cu") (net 2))
 (arc (start 141.1 102.17665) (mid 140.82077 101.502529) (end 140.14665 101.2233) (width 0.2) (layer "F.Cu") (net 2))
 (arc (start 144.83595 109.54735) (mid 144.83595 109.54735) (end 144.83595 109.54735) (width 0.2) (layer "F.Cu") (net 2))
 (arc (start 144.83595 109.54735) (mid 144.83595 109.54735) (end 144.83595 109.54735) (width 0.2) (layer "F.Cu") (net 2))
 (arc (start 154.5 108.25) (mid 153.999999 108.042892) (end 153.499999 108.249999) (width 0.2) (layer "F.Cu") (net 2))
 (arc (start 150.98636 109.4642) (mid 150.98538 109.464394) (end 150.98455 109.46495) (width 0.2) (layer "F.Cu") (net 2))
 (arc (start 147.64695 109.46495) (mid 147.64778 109.465505) (end 147.64876 109.4657) (width 0.2) (layer "F.Cu") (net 2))
 (arc (start 172.75 94.5) (mid 173.305081 95.330737) (end 173.5 96.31066) (width 0.2) (layer "F.Cu") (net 2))
 (arc (start 136.62855 109.4642) (mid 136.463591 109.497012) (end 136.323746 109.590453) (width 0.2) (layer "F.Cu") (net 2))
 (arc (start 136.45 109.28565) (mid 136.502296 109.411903) (end 136.62855 109.4642) (width 0.2) (layer "F.Cu") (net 2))
 (arc (start 144.83595 109.54735) (mid 144.92805 109.485809) (end 145.036691 109.4642) (width 0.2) (layer "F.Cu") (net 2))
 (arc (start 140.6075 109.7482) (mid 140.73787 109.83531) (end 140.891652 109.8659) (width 0.2) (layer "F.Cu") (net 2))
 (segment (start 136.7749 102.7749) (end 135.5 101.5) (width 0.2) (layer "B.Cu") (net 2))
 (segment (start 138.0498 109.4642) (end 138.0498 105.85278) (width 0.2) (layer "B.Cu") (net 2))
 (segment (start 176.866116 105.366116) (end 173.5 102) (width 0.2) (layer "B.Cu") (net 2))
 (segment (start 177.75 107.5) (end 177.75 108.75) (width 0.2) (layer "B.Cu") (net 2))
 (arc (start 176.866116 105.366116) (mid 177.520286 106.34515) (end 177.75 107.5) (width 0.2) (layer "B.Cu") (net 2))
 (arc (start 136.7749 102.7749) (mid 137.718464 104.187043) (end 138.0498 105.85278) (width 0.2) (layer "B.Cu") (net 2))
 (segment (start 160.2638 106.75) (end 160.32505 106.75) (width 0.2) (layer "F.Cu") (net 3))
 (segment (start 151.954531 108.592568) (end 151.8445 108.7026) (width 0.2) (layer "F.Cu") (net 3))
 (segment (start 171.6 92.25) (end 170.1 93.75) (width 0.2) (layer "F.Cu") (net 3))
 (segment (start 160.71065 106.75) (end 161.96 106.75) (width 0.2) (layer "F.Cu") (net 3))
 (segment (start 160.36635 106.75) (end 160.32505 106.75) (width 0.2) (layer "F.Cu") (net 3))
 (segment (start 160.2638 106.75) (end 160.1 106.75) (width 0.2) (layer "F.Cu") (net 3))
 (segment (start 160.66935 106.75) (end 160.62805 106.75) (width 0.2) (layer "F.Cu") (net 3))
 (segment (start 160.548 106.75) (end 160.62805 106.75) (width 0.2) (layer "F.Cu") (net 3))
 (segment (start 160.548 106.75) (end 160.4796 106.75) (width 0.2) (layer "F.Cu") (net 3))
 (segment (start 160.71065 106.75) (end 160.66935 106.75) (width 0.2) (layer "F.Cu") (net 3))
 (segment (start 160.40765 106.75) (end 160.4162 106.75) (width 0.2) (layer "F.Cu") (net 3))
 (segment (start 175.22132 90.75) (end 177.75 90.75) (width 0.2) (layer "F.Cu") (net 3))
 (segment (start 152.319468 107.711531) (end 152.81155 107.21945) (width 0.2) (layer "F.Cu") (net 3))
 (segment (start 160.4746 106.75) (end 160.4162 106.75) (width 0.2) (layer "F.Cu") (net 3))
 (segment (start 160.40765 106.75) (end 160.36635 106.75) (width 0.2) (layer "F.Cu") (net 3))
 (segment (start 147.37255 108.62255) (end 147 108.25) (width 0.2) (layer "F.Cu") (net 3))
 (segment (start 160.4746 106.75) (end 160.4796 106.75) (width 0.2) (layer "F.Cu") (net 3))
 (segment (start 159.069872 106.5449) (end 154.440057 106.5449) (width 0.2) (layer "F.Cu") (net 3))
 (segment (start 148.271965 108.9951) (end 151.138342 108.9951) (width 0.2) (layer "F.Cu") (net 3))
 (segment (start 160.1 106.75) (end 159.565027 106.75) (width 0.2) (layer "F.Cu") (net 3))
 (arc (start 154.440057 106.5449) (mid 153.558715 106.720209) (end 152.81155 107.21945) (width 0.2) (layer "F.Cu") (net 3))
 (arc (start 175.22132 90.75) (mid 173.261475 91.139837) (end 171.6 92.25) (width 0.2) (layer "F.Cu") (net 3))
 (arc (start 159.31745 106.64745) (mid 159.431039 106.723348) (end 159.565027 106.75) (width 0.2) (layer "F.Cu") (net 3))
 (arc (start 159.31745 106.64745) (mid 159.20386 106.571551) (end 159.069872 106.5449) (width 0.2) (layer "F.Cu") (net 3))
 (arc (start 147.37255 108.62255) (mid 147.785205 108.898277) (end 148.271965 108.9951) (width 0.2) (layer "F.Cu") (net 3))
 (arc (start 152.137 108.15205) (mid 152.089577 108.390456) (end 151.954531 108.592568) (width 0.2) (layer "F.Cu") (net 3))
 (arc (start 152.319468 107.711531) (mid 152.184421 107.913642) (end 152.137 108.15205) (width 0.2) (layer "F.Cu") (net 3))
 (arc (start 151.8445 108.7026) (mid 151.520512 108.919081) (end 151.138342 108.9951) (width 0.2) (layer "F.Cu") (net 3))
 (segment (start 176.159009 96.84099) (end 171 102) (width 0.2) (layer "B.Cu") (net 3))
 (segment (start 165.193255 103.516744) (end 161.96 106.75) (width 0.2) (layer "B.Cu") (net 3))
 (segment (start 177.75 93) (end 177.75 90.75) (width 0.2) (layer "B.Cu") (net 3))
 (segment (start 168.855 102) (end 171 102) (width 0.2) (layer "B.Cu") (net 3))
 (arc (start 168.855 102) (mid 166.873278 102.394188) (end 165.193255 103.516744) (width 0.2) (layer "B.Cu") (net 3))
 (arc (start 177.75 93) (mid 177.336514 95.078728) (end 176.159009 96.84099) (width 0.2) (layer "B.Cu") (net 3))
 (segment (start 144.76875 93.5) (end 145.30625 93.5) (width 0.2) (layer "F.Cu") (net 4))
 (segment (start 149.358391 93.5) (end 145.30625 93.5) (width 0.2) (layer "F.Cu") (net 4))
 (segment (start 143.75 107.5) (end 143 108.25) (width 0.2) (layer "F.Cu") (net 4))
 (segment (start 151.776708 92.4983) (end 158.624077 92.4983) (width 0.2) (layer "F.Cu") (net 4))
 (segment (start 164.62415 95.5) (end 165.5 95.5) (width 0.2) (layer "F.Cu") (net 4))
 (segment (start 144.5 103.13) (end 144.5 94.417569) (width 0.2) (layer "F.Cu") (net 4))
 (segment (start 144.5 105.689339) (end 144.5 103.13) (width 0.2) (layer "F.Cu") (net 4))
 (segment (start 162.24745 93.99915) (end 163.12898 94.88068) (width 0.2) (layer "F.Cu") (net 4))
 (segment (start 144.76875 93.5) (end 144.5 93.5) (width 0.2) (layer "F.Cu") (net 4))
 (segment (start 144.768749 93.768749) (end 144.847465 93.690034) (width 0.2) (layer "F.Cu") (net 4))
 (arc (start 163.12898 94.88068) (mid 163.814969 95.339043) (end 164.62415 95.5) (width 0.2) (layer "F.Cu") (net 4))
 (arc (start 151.776708 92.4983) (mid 151.122316 92.628466) (end 150.56755 92.99915) (width 0.2) (layer "F.Cu") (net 4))
 (arc (start 145.30625 93.5) (mid 145.057957 93.549388) (end 144.847465 93.690034) (width 0.2) (layer "F.Cu") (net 4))
 (arc (start 162.24745 93.99915) (mid 160.585032 92.888358) (end 158.624077 92.4983) (width 0.2) (layer "F.Cu") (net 4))
 (arc (start 144.768749 93.768749) (mid 144.569845 94.06643) (end 144.5 94.417569) (width 0.2) (layer "F.Cu") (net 4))
 (arc (start 150.56755 92.99915) (mid 150.012783 93.369833) (end 149.358391 93.5) (width 0.2) (layer "F.Cu") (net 4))
 (arc (start 144.5 105.689339) (mid 144.305081 106.669261) (end 143.75 107.5) (width 0.2) (layer "F.Cu") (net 4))
 (arc (start 144.847465 93.690034) (mid 144.871596 93.568719) (end 144.76875 93.5) (width 0.2) (layer "F.Cu") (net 4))
 (segment (start 151.075 106.00045) (end 151.075 107.75) (width 0.2) (layer "F.Cu") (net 1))
 (segment (start 162.67203 105.6792) (end 151.39625 105.6792) (width 0.2) (layer "F.Cu") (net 1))
 (segment (start 147.9 104.08335) (end 147.9 103.13) (width 0.2) (layer "F.Cu") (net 1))
 (segment (start 150.75375 105.0367) (end 148.85335 105.0367) (width 0.2) (layer "F.Cu") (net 1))
 (segment (start 163.9646 106.2146) (end 164.5 106.75) (width 0.2) (layer "F.Cu") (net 1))
 (segment (start 151.075 106.00045) (end 151.075 105.35795) (width 0.2) (layer "F.Cu") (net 1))
 (arc (start 151.075 105.35795) (mid 150.980908 105.130791) (end 150.75375 105.0367) (width 0.2) (layer "F.Cu") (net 1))
 (arc (start 163.9646 106.2146) (mid 163.371563 105.818345) (end 162.67203 105.6792) (width 0.2) (layer "F.Cu") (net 1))
 (arc (start 151.39625 105.6792) (mid 151.169091 105.773291) (end 151.075 106.00045) (width 0.2) (layer "F.Cu") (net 1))
 (arc (start 151.075 105.35795) (mid 151.169091 105.585108) (end 151.39625 105.6792) (width 0.2) (layer "F.Cu") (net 1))
 (arc (start 147.9 104.08335) (mid 148.179229 104.75747) (end 148.85335 105.0367) (width 0.2) (layer "F.Cu") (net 1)))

